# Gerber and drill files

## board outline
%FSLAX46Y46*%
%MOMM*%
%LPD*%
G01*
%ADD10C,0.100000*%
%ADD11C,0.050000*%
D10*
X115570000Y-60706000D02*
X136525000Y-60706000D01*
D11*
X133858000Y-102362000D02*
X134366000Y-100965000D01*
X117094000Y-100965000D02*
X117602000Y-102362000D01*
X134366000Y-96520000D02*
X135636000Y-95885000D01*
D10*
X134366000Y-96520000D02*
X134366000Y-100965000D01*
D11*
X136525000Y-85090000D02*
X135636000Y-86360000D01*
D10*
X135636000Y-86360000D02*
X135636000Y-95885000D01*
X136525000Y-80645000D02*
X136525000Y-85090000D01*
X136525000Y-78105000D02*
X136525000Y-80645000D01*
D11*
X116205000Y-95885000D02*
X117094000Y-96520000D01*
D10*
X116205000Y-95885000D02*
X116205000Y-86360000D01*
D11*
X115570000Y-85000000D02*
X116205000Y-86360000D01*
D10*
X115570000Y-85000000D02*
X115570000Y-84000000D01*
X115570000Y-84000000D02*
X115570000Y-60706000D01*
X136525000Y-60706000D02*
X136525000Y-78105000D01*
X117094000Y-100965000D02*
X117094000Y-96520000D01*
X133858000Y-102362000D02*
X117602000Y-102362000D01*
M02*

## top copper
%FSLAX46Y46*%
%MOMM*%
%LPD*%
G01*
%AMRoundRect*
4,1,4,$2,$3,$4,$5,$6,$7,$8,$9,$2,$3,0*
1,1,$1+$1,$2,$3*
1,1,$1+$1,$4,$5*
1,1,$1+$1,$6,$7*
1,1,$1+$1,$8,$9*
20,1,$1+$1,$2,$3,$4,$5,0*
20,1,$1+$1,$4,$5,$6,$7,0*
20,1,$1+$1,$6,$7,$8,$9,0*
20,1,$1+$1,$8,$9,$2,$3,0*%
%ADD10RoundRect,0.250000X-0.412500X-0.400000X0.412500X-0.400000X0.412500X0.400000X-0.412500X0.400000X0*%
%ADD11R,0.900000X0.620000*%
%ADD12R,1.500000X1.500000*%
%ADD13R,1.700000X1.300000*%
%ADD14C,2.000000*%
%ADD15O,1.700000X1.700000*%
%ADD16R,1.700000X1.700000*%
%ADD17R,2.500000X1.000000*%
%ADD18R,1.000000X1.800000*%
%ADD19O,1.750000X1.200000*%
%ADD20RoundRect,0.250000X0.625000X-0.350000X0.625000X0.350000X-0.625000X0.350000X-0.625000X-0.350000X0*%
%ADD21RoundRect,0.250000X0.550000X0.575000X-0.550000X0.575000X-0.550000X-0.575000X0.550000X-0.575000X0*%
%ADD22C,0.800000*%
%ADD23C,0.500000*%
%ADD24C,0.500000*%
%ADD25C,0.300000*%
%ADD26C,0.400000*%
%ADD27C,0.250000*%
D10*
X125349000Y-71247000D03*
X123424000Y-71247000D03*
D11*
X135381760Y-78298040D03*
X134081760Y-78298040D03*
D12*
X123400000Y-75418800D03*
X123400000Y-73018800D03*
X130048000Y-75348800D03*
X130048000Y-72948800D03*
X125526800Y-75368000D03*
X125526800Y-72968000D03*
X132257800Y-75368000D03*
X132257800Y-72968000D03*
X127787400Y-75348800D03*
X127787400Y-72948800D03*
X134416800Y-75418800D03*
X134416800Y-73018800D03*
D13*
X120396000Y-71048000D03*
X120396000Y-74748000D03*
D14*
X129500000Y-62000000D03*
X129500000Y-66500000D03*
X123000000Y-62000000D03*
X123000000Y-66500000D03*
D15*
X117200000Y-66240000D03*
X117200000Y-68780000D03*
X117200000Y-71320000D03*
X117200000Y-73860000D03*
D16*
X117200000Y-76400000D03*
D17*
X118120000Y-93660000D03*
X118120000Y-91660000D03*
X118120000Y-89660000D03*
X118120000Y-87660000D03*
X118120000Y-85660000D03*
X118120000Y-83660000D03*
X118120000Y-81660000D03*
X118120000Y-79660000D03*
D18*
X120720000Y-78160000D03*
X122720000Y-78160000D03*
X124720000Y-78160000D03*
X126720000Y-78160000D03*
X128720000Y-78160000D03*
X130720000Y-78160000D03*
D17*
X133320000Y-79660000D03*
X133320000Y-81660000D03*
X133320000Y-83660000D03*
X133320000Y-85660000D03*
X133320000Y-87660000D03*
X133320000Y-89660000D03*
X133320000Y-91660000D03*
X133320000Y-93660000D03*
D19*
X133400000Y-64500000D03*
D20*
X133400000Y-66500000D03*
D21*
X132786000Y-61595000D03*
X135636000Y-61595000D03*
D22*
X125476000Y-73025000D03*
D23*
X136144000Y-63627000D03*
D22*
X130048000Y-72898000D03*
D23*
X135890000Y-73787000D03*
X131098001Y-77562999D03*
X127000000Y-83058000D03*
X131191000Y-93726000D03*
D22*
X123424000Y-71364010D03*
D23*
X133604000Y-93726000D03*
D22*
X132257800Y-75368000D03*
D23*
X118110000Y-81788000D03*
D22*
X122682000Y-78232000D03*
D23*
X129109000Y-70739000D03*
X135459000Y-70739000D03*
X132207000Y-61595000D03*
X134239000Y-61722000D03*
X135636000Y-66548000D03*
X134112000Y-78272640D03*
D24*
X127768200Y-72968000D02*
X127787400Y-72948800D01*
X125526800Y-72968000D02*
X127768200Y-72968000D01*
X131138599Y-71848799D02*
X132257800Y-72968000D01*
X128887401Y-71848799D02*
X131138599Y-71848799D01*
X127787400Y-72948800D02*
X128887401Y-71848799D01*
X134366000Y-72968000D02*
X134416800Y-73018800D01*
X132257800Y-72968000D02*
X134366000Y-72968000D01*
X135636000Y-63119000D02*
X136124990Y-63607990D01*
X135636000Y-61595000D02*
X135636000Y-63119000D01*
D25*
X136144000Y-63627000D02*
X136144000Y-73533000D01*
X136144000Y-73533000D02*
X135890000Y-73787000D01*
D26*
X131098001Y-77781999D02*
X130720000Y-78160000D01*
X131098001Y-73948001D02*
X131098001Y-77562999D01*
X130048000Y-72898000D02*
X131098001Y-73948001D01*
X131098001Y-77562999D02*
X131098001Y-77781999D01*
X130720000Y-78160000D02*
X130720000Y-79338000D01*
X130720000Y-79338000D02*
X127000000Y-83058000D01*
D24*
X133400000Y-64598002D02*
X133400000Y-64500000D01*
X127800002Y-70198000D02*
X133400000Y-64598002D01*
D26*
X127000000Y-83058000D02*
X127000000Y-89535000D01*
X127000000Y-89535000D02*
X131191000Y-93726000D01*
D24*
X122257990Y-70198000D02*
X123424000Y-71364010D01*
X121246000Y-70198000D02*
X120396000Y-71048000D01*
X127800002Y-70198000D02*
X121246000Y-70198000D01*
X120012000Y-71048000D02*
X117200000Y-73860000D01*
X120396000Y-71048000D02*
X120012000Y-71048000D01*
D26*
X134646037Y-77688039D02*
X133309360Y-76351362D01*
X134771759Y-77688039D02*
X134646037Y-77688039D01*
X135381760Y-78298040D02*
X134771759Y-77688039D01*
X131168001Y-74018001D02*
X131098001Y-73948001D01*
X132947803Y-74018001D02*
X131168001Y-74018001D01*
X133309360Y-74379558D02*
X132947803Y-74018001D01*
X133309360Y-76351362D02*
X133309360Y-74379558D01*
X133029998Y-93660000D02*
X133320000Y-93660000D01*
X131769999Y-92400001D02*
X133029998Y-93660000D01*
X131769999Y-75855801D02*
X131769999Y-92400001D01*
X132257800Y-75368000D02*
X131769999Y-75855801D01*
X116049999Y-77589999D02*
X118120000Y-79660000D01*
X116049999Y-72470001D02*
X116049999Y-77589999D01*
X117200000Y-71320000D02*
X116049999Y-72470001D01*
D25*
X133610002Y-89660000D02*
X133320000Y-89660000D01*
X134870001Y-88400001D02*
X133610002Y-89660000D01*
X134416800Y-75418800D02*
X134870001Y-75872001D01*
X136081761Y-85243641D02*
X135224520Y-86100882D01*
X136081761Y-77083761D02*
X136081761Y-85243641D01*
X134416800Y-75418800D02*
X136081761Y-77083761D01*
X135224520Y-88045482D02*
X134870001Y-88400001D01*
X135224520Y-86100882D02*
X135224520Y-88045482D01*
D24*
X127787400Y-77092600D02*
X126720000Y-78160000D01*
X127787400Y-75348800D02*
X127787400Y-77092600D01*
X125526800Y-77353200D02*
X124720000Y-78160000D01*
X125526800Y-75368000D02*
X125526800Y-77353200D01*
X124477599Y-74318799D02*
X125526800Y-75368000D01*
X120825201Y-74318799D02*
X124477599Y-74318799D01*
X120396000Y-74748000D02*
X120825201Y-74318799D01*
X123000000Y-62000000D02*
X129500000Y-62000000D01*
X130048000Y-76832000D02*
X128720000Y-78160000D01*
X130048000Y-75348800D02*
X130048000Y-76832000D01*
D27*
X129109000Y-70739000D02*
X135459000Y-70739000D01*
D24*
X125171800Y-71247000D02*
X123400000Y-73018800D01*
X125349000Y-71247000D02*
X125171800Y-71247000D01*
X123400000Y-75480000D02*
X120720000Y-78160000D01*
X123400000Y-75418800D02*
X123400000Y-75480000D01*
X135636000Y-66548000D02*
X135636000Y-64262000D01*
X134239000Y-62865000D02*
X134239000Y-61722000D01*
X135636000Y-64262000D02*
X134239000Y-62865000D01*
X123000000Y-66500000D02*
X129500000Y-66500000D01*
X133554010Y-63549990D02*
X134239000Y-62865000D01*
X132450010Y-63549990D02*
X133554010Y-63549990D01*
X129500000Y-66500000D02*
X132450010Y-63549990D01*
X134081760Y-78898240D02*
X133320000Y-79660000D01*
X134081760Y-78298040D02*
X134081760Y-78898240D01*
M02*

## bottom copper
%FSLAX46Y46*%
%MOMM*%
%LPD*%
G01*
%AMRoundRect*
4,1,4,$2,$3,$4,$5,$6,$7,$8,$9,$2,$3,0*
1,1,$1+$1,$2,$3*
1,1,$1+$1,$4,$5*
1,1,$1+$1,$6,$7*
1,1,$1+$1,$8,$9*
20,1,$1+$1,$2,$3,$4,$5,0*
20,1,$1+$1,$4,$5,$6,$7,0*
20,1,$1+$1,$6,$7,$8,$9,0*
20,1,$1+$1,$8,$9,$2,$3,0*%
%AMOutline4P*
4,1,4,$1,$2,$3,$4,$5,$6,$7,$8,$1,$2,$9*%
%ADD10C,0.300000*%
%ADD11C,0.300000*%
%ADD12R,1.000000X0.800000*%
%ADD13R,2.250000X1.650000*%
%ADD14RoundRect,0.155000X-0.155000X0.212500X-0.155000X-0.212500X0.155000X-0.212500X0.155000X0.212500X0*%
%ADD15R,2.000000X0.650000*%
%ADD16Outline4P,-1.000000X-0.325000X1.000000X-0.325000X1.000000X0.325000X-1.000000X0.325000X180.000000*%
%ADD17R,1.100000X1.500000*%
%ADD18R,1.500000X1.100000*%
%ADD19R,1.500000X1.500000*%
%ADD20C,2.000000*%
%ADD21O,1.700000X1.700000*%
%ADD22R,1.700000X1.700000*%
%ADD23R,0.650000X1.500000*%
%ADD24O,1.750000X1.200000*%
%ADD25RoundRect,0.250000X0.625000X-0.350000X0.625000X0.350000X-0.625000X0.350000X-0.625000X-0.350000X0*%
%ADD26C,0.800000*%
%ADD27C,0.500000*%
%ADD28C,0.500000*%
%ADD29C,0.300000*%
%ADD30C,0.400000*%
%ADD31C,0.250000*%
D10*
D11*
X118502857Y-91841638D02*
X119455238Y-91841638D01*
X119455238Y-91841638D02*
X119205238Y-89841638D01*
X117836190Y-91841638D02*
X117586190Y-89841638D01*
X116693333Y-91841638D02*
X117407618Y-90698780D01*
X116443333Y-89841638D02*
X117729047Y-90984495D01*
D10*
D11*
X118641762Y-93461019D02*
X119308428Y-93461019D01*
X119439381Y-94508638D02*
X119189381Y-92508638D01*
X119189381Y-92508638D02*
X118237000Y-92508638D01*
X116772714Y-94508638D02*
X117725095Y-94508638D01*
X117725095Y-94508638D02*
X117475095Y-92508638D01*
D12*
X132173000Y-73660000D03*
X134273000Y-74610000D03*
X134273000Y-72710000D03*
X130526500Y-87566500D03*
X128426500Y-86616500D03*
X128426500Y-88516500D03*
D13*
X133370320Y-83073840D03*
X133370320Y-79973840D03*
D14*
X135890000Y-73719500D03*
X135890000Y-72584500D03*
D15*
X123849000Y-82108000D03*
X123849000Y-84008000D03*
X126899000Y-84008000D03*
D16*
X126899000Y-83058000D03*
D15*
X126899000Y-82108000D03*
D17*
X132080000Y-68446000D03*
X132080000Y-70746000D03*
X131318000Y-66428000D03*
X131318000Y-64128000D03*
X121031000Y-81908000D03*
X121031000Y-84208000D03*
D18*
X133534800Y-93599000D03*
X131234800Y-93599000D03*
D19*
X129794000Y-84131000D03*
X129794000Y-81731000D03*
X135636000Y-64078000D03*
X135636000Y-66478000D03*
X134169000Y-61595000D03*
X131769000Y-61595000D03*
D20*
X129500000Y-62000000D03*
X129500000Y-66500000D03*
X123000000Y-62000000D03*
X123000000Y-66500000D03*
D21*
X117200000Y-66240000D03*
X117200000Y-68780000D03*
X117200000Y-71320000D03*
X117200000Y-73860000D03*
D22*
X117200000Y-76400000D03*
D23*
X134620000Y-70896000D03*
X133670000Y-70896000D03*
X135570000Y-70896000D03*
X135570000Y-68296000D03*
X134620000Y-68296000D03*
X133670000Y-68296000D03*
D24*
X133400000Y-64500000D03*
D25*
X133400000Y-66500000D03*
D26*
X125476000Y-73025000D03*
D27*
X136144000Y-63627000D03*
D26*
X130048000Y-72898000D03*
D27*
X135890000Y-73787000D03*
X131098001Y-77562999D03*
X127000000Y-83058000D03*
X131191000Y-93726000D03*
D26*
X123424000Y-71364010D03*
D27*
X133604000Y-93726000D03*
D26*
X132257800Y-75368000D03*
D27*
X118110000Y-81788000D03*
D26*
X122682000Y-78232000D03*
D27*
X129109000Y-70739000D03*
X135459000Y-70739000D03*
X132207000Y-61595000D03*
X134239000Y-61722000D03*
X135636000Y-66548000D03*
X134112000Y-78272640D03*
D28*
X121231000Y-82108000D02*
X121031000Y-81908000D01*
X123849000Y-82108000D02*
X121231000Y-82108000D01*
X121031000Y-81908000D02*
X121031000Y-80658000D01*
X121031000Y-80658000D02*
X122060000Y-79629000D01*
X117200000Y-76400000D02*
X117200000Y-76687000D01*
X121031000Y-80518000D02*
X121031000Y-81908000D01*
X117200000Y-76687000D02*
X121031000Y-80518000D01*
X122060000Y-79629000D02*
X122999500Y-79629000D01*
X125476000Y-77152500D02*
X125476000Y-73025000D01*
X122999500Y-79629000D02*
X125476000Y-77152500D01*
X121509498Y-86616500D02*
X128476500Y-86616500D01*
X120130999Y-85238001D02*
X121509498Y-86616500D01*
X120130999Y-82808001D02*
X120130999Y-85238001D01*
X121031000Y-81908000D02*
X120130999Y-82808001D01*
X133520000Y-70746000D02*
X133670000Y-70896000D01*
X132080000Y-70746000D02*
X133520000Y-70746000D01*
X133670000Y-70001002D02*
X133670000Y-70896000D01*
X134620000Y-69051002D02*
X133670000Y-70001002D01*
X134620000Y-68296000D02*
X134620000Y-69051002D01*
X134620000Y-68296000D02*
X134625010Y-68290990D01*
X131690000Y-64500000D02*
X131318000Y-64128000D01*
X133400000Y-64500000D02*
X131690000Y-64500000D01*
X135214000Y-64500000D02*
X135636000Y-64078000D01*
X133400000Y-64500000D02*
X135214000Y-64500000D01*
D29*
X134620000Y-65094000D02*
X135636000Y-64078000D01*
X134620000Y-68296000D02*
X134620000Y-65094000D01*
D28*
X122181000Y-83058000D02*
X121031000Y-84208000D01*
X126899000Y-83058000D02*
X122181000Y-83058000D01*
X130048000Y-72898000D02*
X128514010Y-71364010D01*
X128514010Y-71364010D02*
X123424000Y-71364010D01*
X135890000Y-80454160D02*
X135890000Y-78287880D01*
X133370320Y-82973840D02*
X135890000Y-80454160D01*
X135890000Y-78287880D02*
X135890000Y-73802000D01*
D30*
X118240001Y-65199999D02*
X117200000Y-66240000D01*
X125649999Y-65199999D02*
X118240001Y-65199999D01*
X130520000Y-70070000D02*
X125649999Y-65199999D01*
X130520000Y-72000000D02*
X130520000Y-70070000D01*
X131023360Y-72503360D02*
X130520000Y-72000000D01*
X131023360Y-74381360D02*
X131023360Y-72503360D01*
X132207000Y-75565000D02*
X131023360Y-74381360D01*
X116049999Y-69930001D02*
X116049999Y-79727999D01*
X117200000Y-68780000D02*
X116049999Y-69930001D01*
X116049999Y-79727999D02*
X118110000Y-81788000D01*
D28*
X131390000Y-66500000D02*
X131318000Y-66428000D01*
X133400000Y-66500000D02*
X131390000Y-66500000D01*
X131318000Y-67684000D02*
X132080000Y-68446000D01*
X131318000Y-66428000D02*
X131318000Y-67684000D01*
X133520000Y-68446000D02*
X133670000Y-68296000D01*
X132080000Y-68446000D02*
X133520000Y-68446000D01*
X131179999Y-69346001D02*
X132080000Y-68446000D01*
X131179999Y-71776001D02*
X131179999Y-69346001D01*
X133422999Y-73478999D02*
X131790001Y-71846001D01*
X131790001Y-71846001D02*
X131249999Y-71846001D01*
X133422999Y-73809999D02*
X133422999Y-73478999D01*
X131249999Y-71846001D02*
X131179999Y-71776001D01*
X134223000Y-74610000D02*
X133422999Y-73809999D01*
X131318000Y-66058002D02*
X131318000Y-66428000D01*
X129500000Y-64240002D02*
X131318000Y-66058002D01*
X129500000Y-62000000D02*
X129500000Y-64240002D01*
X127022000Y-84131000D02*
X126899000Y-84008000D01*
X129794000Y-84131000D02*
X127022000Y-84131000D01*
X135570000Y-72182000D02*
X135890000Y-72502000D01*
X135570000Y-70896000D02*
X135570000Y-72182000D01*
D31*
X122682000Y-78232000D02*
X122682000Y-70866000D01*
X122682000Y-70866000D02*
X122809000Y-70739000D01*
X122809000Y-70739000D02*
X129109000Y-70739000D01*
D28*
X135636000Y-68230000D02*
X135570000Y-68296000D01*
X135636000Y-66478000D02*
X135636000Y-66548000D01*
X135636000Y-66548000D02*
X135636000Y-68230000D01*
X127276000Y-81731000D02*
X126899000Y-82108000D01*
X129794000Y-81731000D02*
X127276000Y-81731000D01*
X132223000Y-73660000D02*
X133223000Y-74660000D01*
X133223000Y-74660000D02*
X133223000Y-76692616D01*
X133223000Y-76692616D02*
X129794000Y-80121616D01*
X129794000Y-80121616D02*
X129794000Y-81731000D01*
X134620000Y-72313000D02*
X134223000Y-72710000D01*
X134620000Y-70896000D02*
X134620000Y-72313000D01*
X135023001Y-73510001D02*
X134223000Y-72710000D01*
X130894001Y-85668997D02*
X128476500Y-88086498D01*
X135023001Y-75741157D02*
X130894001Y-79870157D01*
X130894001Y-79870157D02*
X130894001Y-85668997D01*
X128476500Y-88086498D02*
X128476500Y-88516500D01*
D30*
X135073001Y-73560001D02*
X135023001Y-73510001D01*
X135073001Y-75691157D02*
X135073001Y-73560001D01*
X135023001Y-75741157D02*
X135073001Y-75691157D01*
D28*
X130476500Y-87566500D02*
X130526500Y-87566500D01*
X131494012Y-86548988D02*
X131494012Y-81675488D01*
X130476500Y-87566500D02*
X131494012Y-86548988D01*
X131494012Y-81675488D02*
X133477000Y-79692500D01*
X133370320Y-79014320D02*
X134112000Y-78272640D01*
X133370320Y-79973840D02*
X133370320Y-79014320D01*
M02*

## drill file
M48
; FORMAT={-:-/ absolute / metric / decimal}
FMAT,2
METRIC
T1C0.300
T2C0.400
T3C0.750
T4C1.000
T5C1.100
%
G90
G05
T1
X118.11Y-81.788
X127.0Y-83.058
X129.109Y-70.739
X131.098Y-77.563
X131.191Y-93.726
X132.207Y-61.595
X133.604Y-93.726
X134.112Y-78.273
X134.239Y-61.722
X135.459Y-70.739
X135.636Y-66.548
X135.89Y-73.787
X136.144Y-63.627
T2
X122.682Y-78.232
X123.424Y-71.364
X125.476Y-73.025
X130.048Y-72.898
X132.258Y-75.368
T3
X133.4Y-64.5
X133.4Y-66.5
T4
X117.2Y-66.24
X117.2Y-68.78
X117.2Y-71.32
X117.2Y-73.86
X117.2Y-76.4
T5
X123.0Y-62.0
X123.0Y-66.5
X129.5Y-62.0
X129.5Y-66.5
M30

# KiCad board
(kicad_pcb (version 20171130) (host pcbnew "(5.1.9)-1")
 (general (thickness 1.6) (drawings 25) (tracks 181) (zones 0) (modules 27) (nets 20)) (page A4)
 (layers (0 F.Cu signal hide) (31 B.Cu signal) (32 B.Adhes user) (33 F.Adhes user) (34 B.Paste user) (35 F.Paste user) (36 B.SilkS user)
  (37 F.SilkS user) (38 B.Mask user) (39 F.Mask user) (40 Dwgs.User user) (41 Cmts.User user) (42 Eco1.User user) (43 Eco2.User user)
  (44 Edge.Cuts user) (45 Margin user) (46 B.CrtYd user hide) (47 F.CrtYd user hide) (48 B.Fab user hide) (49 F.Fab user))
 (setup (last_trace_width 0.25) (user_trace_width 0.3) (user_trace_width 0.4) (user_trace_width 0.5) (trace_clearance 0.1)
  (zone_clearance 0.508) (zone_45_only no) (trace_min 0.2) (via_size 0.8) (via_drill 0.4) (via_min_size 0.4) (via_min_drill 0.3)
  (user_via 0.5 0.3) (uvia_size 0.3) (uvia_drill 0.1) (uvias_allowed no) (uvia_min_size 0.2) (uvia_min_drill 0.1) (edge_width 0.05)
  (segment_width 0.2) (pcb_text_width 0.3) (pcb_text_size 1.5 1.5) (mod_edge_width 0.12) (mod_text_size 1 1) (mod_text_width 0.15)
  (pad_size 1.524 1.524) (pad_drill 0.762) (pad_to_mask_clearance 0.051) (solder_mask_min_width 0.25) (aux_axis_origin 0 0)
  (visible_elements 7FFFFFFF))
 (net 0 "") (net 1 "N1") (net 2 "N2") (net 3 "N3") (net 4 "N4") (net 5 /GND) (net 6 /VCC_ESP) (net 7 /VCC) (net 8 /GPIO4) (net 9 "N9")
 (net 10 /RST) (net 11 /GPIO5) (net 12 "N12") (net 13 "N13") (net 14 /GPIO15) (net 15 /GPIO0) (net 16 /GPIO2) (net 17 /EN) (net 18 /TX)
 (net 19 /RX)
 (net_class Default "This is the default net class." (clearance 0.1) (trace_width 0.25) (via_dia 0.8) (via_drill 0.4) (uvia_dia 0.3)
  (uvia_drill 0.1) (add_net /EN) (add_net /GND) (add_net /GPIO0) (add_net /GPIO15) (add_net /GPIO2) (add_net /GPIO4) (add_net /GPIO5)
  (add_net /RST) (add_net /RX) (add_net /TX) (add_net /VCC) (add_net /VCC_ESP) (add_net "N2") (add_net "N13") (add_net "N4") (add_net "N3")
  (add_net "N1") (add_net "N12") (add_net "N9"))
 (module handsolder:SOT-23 (layer B.Cu) (at 133.223 73.66 180)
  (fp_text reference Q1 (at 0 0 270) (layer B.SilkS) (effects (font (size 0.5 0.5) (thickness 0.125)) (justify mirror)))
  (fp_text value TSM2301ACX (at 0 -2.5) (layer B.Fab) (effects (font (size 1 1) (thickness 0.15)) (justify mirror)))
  (pad 3 smd rect (at 1.05 0 180) (size 1 0.8) (layers B.Cu B.Paste B.Mask) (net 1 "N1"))
  (pad 2 smd rect (at -1.05 -0.95 180) (size 1 0.8) (layers B.Cu B.Paste B.Mask) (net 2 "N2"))
  (pad 1 smd rect (at -1.05 0.95 180) (size 1 0.8) (layers B.Cu B.Paste B.Mask) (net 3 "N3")))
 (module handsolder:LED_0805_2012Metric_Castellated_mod (layer F.Cu) (at 124.3865 71.247)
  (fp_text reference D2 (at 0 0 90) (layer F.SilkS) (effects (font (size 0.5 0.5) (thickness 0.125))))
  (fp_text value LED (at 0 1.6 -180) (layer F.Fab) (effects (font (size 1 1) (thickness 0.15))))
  (pad 2 smd roundrect (at 0.9625 0) (size 1.325 1.3) (layers F.Cu F.Paste F.Mask) (roundrect_rratio 0.1923076923076923) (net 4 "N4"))
  (pad 1 smd roundrect (at -0.9625 0) (size 1.325 1.3) (layers F.Cu F.Paste F.Mask) (roundrect_rratio 0.1923076923076923) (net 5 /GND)))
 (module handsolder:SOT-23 (layer B.Cu) (at 129.4765 87.5665)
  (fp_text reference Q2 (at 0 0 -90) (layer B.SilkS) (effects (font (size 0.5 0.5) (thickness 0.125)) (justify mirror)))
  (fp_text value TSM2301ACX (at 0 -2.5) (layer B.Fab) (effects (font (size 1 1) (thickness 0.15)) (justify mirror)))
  (pad 3 smd rect (at 1.05 0) (size 1 0.8) (layers B.Cu B.Paste B.Mask) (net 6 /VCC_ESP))
  (pad 2 smd rect (at -1.05 -0.95) (size 1 0.8) (layers B.Cu B.Paste B.Mask) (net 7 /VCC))
  (pad 1 smd rect (at -1.05 0.95) (size 1 0.8) (layers B.Cu B.Paste B.Mask) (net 3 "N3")))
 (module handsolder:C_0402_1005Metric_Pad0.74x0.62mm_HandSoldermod (layer F.Cu) (at 134.73176 78.29804)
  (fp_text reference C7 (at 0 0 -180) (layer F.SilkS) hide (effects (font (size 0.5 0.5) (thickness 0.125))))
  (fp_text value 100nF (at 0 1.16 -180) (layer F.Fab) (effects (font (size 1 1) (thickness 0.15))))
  (pad 2 smd rect (at 0.65 0) (size 0.9 0.62) (layers F.Cu F.Paste F.Mask) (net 5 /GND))
  (pad 1 smd rect (at -0.65 0) (size 0.9 0.62) (layers F.Cu F.Paste F.Mask) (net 6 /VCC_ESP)))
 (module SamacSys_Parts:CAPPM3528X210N (layer B.Cu) (at 133.37032 81.52384 270)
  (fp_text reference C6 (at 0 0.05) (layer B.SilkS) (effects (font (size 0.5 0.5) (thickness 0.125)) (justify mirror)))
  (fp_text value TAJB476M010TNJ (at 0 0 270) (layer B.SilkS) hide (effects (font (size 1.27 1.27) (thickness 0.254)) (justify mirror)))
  (pad 2 smd rect (at 1.55 0 270) (size 1.65 2.25) (layers B.Cu B.Paste B.Mask) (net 5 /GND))
  (pad 1 smd rect (at -1.55 0 270) (size 1.65 2.25) (layers B.Cu B.Paste B.Mask) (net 6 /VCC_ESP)))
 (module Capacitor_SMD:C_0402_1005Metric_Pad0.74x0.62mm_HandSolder (layer B.Cu) (at 135.89 73.152 270)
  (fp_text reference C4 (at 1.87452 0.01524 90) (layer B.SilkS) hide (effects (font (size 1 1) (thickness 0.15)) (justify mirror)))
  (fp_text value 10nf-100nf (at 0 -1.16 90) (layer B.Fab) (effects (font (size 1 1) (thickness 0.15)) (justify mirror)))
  (pad 2 smd roundrect (at 0.5675 0 270) (size 0.735 0.62) (layers B.Cu B.Paste B.Mask) (roundrect_rratio 0.25) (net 5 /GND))
  (pad 1 smd roundrect (at -0.5675 0 270) (size 0.735 0.62) (layers B.Cu B.Paste B.Mask) (roundrect_rratio 0.25) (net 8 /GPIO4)))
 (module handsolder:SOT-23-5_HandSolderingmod (layer B.Cu) (at 125.349 83.058 180)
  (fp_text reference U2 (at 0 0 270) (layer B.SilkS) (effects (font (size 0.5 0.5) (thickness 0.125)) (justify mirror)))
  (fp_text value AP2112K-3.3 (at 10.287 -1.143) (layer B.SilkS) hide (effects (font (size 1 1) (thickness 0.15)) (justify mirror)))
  (pad 5 smd rect (at 1.5 0.95 180) (size 2 0.65) (layers B.Cu B.Paste B.Mask) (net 7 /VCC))
  (pad 4 smd rect (at 1.5 -0.95 180) (size 2 0.65) (layers B.Cu B.Paste B.Mask))
  (pad 3 smd rect (at -1.55 -0.95 180) (size 2 0.65) (layers B.Cu B.Paste B.Mask) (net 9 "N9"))
  (pad 2 smd trapezoid (at -1.55 0 180) (size 2 0.65) (layers B.Cu B.Paste B.Mask) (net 5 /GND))
  (pad 1 smd rect (at -1.55 0.95 180) (size 2 0.65) (layers B.Cu B.Paste B.Mask) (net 1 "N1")))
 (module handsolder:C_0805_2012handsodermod (layer B.Cu) (at 132.08 69.596 90)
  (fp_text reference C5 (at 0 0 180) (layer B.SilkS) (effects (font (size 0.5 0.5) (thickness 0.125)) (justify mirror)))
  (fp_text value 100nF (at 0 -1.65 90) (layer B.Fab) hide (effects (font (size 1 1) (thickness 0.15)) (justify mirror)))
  (pad 2 smd rect (at 1.15 0 90) (size 1.5 1.1) (layers B.Cu B.Paste B.Mask) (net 2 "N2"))
  (pad 1 smd rect (at -1.15 0 90) (size 1.5 1.1) (layers B.Cu B.Paste B.Mask) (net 5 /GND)))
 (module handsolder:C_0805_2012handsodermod (layer B.Cu) (at 131.318 65.278 270)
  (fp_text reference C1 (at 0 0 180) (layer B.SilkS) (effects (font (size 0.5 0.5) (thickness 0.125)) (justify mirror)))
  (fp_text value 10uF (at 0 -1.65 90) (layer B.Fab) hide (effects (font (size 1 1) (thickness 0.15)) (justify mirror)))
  (pad 2 smd rect (at 1.15 0 270) (size 1.5 1.1) (layers B.Cu B.Paste B.Mask) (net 2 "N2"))
  (pad 1 smd rect (at -1.15 0 270) (size 1.5 1.1) (layers B.Cu B.Paste B.Mask) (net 5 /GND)))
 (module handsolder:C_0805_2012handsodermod (layer B.Cu) (at 121.031 83.058 90)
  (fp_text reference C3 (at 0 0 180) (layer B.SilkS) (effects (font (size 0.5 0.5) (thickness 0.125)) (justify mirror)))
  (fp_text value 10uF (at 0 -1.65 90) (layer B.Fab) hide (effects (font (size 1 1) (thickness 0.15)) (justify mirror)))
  (pad 2 smd rect (at 1.15 0 90) (size 1.5 1.1) (layers B.Cu B.Paste B.Mask) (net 7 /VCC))
  (pad 1 smd rect (at -1.15 0 90) (size 1.5 1.1) (layers B.Cu B.Paste B.Mask) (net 5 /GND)))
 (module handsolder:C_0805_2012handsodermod (layer B.Cu) (at 132.3848 93.599)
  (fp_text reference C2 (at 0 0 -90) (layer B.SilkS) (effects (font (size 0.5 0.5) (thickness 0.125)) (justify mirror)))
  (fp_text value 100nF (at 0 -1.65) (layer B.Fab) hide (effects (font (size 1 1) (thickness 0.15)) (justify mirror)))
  (pad 2 smd rect (at 1.15 0) (size 1.5 1.1) (layers B.Cu B.Paste B.Mask) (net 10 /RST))
  (pad 1 smd rect (at -1.15 0) (size 1.5 1.1) (layers B.Cu B.Paste B.Mask) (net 5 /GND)))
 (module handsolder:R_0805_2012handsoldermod (layer F.Cu) (at 123.4 74.2188 270)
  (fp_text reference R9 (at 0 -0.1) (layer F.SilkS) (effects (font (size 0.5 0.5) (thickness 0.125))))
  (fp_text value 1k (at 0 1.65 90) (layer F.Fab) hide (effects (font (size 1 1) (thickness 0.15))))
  (pad 2 smd rect (at 1.2 0 270) (size 1.5 1.5) (layers F.Cu F.Paste F.Mask) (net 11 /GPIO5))
  (pad 1 smd rect (at -1.2 0 270) (size 1.5 1.5) (layers F.Cu F.Paste F.Mask) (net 4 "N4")))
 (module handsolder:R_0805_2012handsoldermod (layer B.Cu) (at 129.794 82.931 270)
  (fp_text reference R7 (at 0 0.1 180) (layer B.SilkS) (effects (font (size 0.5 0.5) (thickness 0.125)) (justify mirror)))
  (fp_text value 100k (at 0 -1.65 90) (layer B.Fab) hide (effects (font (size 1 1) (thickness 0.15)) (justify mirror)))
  (pad 2 smd rect (at 1.2 0 270) (size 1.5 1.5) (layers B.Cu B.Paste B.Mask) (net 9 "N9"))
  (pad 1 smd rect (at -1.2 0 270) (size 1.5 1.5) (layers B.Cu B.Paste B.Mask) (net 1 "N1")))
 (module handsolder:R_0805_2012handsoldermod (layer B.Cu) (at 135.636 65.278 90)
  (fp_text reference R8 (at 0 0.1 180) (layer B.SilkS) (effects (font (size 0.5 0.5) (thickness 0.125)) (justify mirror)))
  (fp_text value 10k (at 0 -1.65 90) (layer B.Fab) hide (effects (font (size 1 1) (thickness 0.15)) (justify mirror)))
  (pad 2 smd rect (at 1.2 0 90) (size 1.5 1.5) (layers B.Cu B.Paste B.Mask) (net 5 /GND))
  (pad 1 smd rect (at -1.2 0 90) (size 1.5 1.5) (layers B.Cu B.Paste B.Mask) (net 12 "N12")))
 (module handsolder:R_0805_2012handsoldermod (layer B.Cu) (at 132.969 61.595)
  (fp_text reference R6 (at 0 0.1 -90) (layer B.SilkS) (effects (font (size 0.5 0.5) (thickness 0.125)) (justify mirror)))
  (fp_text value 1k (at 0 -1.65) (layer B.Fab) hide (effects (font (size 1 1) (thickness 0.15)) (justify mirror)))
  (pad 2 smd rect (at 1.2 0) (size 1.5 1.5) (layers B.Cu B.Paste B.Mask) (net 12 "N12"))
  (pad 1 smd rect (at -1.2 0) (size 1.5 1.5) (layers B.Cu B.Paste B.Mask) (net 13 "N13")))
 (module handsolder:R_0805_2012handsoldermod (layer F.Cu) (at 130.048 74.1488 270)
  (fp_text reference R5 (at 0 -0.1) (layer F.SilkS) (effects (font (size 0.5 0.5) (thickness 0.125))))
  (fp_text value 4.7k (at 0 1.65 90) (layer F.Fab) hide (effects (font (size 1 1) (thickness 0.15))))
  (pad 2 smd rect (at 1.2 0 270) (size 1.5 1.5) (layers F.Cu F.Paste F.Mask) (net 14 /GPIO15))
  (pad 1 smd rect (at -1.2 0 270) (size 1.5 1.5) (layers F.Cu F.Paste F.Mask) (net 5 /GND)))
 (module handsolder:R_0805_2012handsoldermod (layer F.Cu) (at 125.5268 74.168 270)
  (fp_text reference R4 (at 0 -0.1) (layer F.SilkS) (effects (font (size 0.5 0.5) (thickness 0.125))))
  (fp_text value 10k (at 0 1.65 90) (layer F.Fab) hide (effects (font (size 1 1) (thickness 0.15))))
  (pad 2 smd rect (at 1.2 0 270) (size 1.5 1.5) (layers F.Cu F.Paste F.Mask) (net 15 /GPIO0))
  (pad 1 smd rect (at -1.2 0 270) (size 1.5 1.5) (layers F.Cu F.Paste F.Mask) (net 7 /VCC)))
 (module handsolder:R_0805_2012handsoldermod (layer F.Cu) (at 132.2578 74.168 270)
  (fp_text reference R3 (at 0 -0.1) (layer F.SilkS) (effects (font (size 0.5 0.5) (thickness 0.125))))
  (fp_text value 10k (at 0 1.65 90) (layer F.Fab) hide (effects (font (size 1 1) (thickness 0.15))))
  (pad 2 smd rect (at 1.2 0 270) (size 1.5 1.5) (layers F.Cu F.Paste F.Mask) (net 10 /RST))
  (pad 1 smd rect (at -1.2 0 270) (size 1.5 1.5) (layers F.Cu F.Paste F.Mask) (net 7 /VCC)))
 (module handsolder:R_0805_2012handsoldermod (layer F.Cu) (at 127.7874 74.1488 270)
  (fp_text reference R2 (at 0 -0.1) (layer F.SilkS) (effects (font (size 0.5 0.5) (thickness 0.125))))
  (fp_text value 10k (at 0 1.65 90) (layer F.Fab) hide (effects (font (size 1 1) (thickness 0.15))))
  (pad 2 smd rect (at 1.2 0 270) (size 1.5 1.5) (layers F.Cu F.Paste F.Mask) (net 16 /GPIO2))
  (pad 1 smd rect (at -1.2 0 270) (size 1.5 1.5) (layers F.Cu F.Paste F.Mask) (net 7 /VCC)))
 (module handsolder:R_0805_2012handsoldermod (layer F.Cu) (at 134.4168 74.2188 270)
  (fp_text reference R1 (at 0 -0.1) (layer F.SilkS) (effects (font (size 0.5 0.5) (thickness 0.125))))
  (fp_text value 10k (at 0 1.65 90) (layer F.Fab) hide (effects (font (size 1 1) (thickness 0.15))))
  (pad 2 smd rect (at 1.2 0 270) (size 1.5 1.5) (layers F.Cu F.Paste F.Mask) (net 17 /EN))
  (pad 1 smd rect (at -1.2 0 270) (size 1.5 1.5) (layers F.Cu F.Paste F.Mask) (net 7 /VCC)))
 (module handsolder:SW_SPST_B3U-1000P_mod (layer F.Cu) (at 120.396 72.898 90)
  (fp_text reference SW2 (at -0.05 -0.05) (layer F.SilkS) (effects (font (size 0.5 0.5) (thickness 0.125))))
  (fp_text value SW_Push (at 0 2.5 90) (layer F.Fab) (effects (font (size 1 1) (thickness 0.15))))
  (pad 2 smd rect (at 1.85 0 90) (size 1.3 1.7) (layers F.Cu F.Paste F.Mask) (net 5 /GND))
  (pad 1 smd rect (at -1.85 0 90) (size 1.3 1.7) (layers F.Cu F.Paste F.Mask) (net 15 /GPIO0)))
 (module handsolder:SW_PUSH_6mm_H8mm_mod (layer F.Cu) (at 123 62)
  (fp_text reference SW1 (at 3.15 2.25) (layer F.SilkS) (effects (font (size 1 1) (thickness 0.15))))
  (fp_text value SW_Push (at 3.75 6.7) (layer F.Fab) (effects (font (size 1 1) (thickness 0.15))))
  (pad 1 thru_hole circle (at 6.5 0 90) (size 2 2) (drill 1.1) (layers *.Cu *.Mask) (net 2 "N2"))
  (pad 2 thru_hole circle (at 6.5 4.5 90) (size 2 2) (drill 1.1) (layers *.Cu *.Mask) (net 12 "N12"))
  (pad 1 thru_hole circle (at 0 0 90) (size 2 2) (drill 1.1) (layers *.Cu *.Mask) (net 2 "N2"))
  (pad 2 thru_hole circle (at 0 4.5 90) (size 2 2) (drill 1.1) (layers *.Cu *.Mask) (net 12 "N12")))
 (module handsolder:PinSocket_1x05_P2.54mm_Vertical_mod (layer F.Cu) (at 117.2 76.4 180)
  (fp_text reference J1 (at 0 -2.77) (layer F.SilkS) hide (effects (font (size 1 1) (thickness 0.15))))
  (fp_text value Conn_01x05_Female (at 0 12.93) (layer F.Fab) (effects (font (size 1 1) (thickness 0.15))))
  (pad 5 thru_hole oval (at 0 10.16 180) (size 1.7 1.7) (drill 1) (layers *.Cu *.Mask) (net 10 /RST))
  (pad 4 thru_hole oval (at 0 7.62 180) (size 1.7 1.7) (drill 1) (layers *.Cu *.Mask) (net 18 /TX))
  (pad 3 thru_hole oval (at 0 5.08 180) (size 1.7 1.7) (drill 1) (layers *.Cu *.Mask) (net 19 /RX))
  (pad 2 thru_hole oval (at 0 2.54 180) (size 1.7 1.7) (drill 1) (layers *.Cu *.Mask) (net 5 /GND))
  (pad 1 thru_hole rect (at 0 0 180) (size 1.7 1.7) (drill 1) (layers *.Cu *.Mask) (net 7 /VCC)))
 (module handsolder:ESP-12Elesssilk (layer F.Cu) (at 125.72 90.16 180)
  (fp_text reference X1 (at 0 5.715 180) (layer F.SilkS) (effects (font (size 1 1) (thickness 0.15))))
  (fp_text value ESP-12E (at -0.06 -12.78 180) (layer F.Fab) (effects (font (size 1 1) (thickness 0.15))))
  (pad 22 smd rect (at 7.6 -3.5 180) (size 2.5 1) (layers F.Cu F.Paste F.Mask))
  (pad 21 smd rect (at 7.6 -1.5 180) (size 2.5 1) (layers F.Cu F.Paste F.Mask))
  (pad 20 smd rect (at 7.6 0.5 180) (size 2.5 1) (layers F.Cu F.Paste F.Mask))
  (pad 19 smd rect (at 7.6 2.5 180) (size 2.5 1) (layers F.Cu F.Paste F.Mask))
  (pad 18 smd rect (at 7.6 4.5 180) (size 2.5 1) (layers F.Cu F.Paste F.Mask))
  (pad 17 smd rect (at 7.6 6.5 180) (size 2.5 1) (layers F.Cu F.Paste F.Mask))
  (pad 16 smd rect (at 7.6 8.5 180) (size 2.5 1) (layers F.Cu F.Paste F.Mask) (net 18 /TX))
  (pad 15 smd rect (at 7.6 10.5 180) (size 2.5 1) (layers F.Cu F.Paste F.Mask) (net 19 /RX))
  (pad 14 smd rect (at 5 12 180) (size 1 1.8) (layers F.Cu F.Paste F.Mask) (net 11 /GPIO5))
  (pad 13 smd rect (at 3 12 180) (size 1 1.8) (layers F.Cu F.Paste F.Mask) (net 8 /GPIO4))
  (pad 12 smd rect (at 1 12 180) (size 1 1.8) (layers F.Cu F.Paste F.Mask) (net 15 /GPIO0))
  (pad 11 smd rect (at -1 12 180) (size 1 1.8) (layers F.Cu F.Paste F.Mask) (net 16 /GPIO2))
  (pad 10 smd rect (at -3 12 180) (size 1 1.8) (layers F.Cu F.Paste F.Mask) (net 14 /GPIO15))
  (pad 9 smd rect (at -5 12 180) (size 1 1.8) (layers F.Cu F.Paste F.Mask) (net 5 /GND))
  (pad 8 smd rect (at -7.6 10.5 180) (size 2.5 1) (layers F.Cu F.Paste F.Mask) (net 6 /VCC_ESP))
  (pad 7 smd rect (at -7.6 8.5 180) (size 2.5 1) (layers F.Cu F.Paste F.Mask))
  (pad 6 smd rect (at -7.6 6.5 180) (size 2.5 1) (layers F.Cu F.Paste F.Mask))
  (pad 5 smd rect (at -7.6 4.5 180) (size 2.5 1) (layers F.Cu F.Paste F.Mask))
  (pad 4 smd rect (at -7.6 2.5 180) (size 2.5 1) (layers F.Cu F.Paste F.Mask))
  (pad 3 smd rect (at -7.6 0.5 180) (size 2.5 1) (layers F.Cu F.Paste F.Mask) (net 17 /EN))
  (pad 2 smd rect (at -7.6 -1.5 180) (size 2.5 1) (layers F.Cu F.Paste F.Mask))
  (pad 1 smd rect (at -7.6 -3.5 180) (size 2.5 1) (layers F.Cu F.Paste F.Mask) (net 10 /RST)))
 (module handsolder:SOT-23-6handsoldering (layer B.Cu) (at 134.62 69.596 270)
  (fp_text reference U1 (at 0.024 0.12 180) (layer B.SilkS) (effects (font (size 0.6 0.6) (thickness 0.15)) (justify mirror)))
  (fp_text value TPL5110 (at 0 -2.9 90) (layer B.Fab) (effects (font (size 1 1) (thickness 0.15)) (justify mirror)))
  (pad 5 smd rect (at 1.3 0 270) (size 1.5 0.65) (layers B.Cu B.Paste B.Mask) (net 3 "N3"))
  (pad 6 smd rect (at 1.3 0.95 270) (size 1.5 0.65) (layers B.Cu B.Paste B.Mask) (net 5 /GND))
  (pad 4 smd rect (at 1.3 -0.95 270) (size 1.5 0.65) (layers B.Cu B.Paste B.Mask) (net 8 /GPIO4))
  (pad 3 smd rect (at -1.3 -0.95 270) (size 1.5 0.65) (layers B.Cu B.Paste B.Mask) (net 12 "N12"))
  (pad 2 smd rect (at -1.3 0 270) (size 1.5 0.65) (layers B.Cu B.Paste B.Mask) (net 5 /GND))
  (pad 1 smd rect (at -1.3 0.95 270) (size 1.5 0.65) (layers B.Cu B.Paste B.Mask) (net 2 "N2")))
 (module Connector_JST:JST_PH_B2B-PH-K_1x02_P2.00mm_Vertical (layer F.Cu) (at 133.4 66.5 90)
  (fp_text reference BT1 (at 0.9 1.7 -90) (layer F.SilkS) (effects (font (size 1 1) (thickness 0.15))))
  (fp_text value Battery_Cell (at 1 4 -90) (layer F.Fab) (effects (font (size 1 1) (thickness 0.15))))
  (pad 2 thru_hole oval (at 2 0 90) (size 1.2 1.75) (drill 0.75) (layers *.Cu *.Mask) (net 5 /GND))
  (pad 1 thru_hole roundrect (at 0 0 90) (size 1.2 1.75) (drill 0.75) (layers *.Cu *.Mask) (roundrect_rratio 0.208333) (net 2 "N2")))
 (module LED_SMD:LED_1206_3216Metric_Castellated (layer F.Cu) (at 134.211 61.595 180)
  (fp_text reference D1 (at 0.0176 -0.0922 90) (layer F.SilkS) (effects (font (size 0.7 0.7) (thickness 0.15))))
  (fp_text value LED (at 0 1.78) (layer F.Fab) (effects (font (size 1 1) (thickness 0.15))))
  (pad 2 smd roundrect (at 1.425 0 180) (size 1.6 1.65) (layers F.Cu F.Paste F.Mask) (roundrect_rratio 0.15625) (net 13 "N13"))
  (pad 1 smd roundrect (at -1.425 0 180) (size 1.6 1.65) (layers F.Cu F.Paste F.Mask) (roundrect_rratio 0.15625) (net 5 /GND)))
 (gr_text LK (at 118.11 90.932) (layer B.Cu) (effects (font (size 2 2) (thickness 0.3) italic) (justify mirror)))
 (gr_line (start 115.57 60.706) (end 136.525 60.706) (layer Edge.Cuts) (width 0.1))
 (gr_line (start 133.858 102.362) (end 134.366 100.965) (layer Edge.Cuts) (width 0.05))
 (gr_line (start 117.094 100.965) (end 117.602 102.362) (layer Edge.Cuts) (width 0.05))
 (gr_line (start 134.366 96.52) (end 135.636 95.885) (layer Edge.Cuts) (width 0.05))
 (gr_line (start 134.366 96.52) (end 134.366 100.965) (layer Edge.Cuts) (width 0.1))
 (gr_line (start 136.525 85.09) (end 135.636 86.36) (layer Edge.Cuts) (width 0.05))
 (gr_line (start 135.636 86.36) (end 135.636 95.885) (layer Edge.Cuts) (width 0.1))
 (gr_line (start 136.525 80.645) (end 136.525 85.09) (layer Edge.Cuts) (width 0.1))
 (gr_line (start 136.525 78.105) (end 136.525 80.645) (layer Edge.Cuts) (width 0.1))
 (gr_line (start 116.205 95.885) (end 117.094 96.52) (layer Edge.Cuts) (width 0.05))
 (gr_line (start 116.205 95.885) (end 116.205 86.36) (layer Edge.Cuts) (width 0.1))
 (gr_line (start 115.57 85) (end 116.205 86.36) (layer Edge.Cuts) (width 0.05))
 (gr_line (start 115.57 85) (end 115.57 84) (layer Edge.Cuts) (width 0.1))
 (gr_line (start 115.57 84) (end 115.57 60.706) (layer Edge.Cuts) (width 0.1))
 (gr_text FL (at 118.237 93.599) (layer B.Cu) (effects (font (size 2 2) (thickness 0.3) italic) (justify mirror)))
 (gr_line (start 136.525 60.706) (end 136.525 78.105) (layer Edge.Cuts) (width 0.1))
 (gr_line (start 117.094 100.965) (end 117.094 96.52) (layer Edge.Cuts) (width 0.1))
 (gr_line (start 133.858 102.362) (end 117.602 102.362) (layer Edge.Cuts) (width 0.1))
 (via (at 125.476 73.025) (size 0.8) (drill 0.4) (layers F.Cu B.Cu) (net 7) (status 30))
 (segment (start 121.231 82.108) (end 121.031 81.908) (width 0.5) (layer B.Cu) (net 7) (status 30))
 (segment (start 123.849 82.108) (end 121.231 82.108) (width 0.5) (layer B.Cu) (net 7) (status 30))
 (segment (start 121.031 81.908) (end 121.031 80.658) (width 0.5) (layer B.Cu) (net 7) (status 10))
 (segment (start 121.031 80.658) (end 122.06 79.629) (width 0.5) (layer B.Cu) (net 7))
 (segment (start 127.7682 72.968) (end 127.7874 72.9488) (width 0.5) (layer F.Cu) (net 7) (status 30))
 (segment (start 125.5268 72.968) (end 127.7682 72.968) (width 0.5) (layer F.Cu) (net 7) (status 30))
 (segment (start 131.138599 71.848799) (end 132.2578 72.968) (width 0.5) (layer F.Cu) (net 7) (status 20))
 (segment (start 128.887401 71.848799) (end 131.138599 71.848799) (width 0.5) (layer F.Cu) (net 7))
 (segment (start 127.7874 72.9488) (end 128.887401 71.848799) (width 0.5) (layer F.Cu) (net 7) (status 10))
 (segment (start 134.366 72.968) (end 134.4168 73.0188) (width 0.5) (layer F.Cu) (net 7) (status 30))
 (segment (start 132.2578 72.968) (end 134.366 72.968) (width 0.5) (layer F.Cu) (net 7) (status 30))
 (segment (start 117.2 76.4) (end 117.2 76.687) (width 0.5) (layer B.Cu) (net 7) (status 30))
 (segment (start 121.031 80.518) (end 121.031 81.908) (width 0.5) (layer B.Cu) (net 7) (status 20))
 (segment (start 117.2 76.687) (end 121.031 80.518) (width 0.5) (layer B.Cu) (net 7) (status 10))
 (segment (start 122.06 79.629) (end 122.9995 79.629) (width 0.5) (layer B.Cu) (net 7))
 (segment (start 125.476 77.1525) (end 125.476 73.025) (width 0.5) (layer B.Cu) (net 7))
 (segment (start 122.9995 79.629) (end 125.476 77.1525) (width 0.5) (layer B.Cu) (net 7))
 (segment (start 121.509498 86.6165) (end 128.4765 86.6165) (width 0.5) (layer B.Cu) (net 7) (status 20))
 (segment (start 120.130999 85.238001) (end 121.509498 86.6165) (width 0.5) (layer B.Cu) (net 7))
 (segment (start 120.130999 82.808001) (end 120.130999 85.238001) (width 0.5) (layer B.Cu) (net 7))
 (segment (start 121.031 81.908) (end 120.130999 82.808001) (width 0.5) (layer B.Cu) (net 7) (status 10))
 (via (at 136.144 63.627) (size 0.5) (drill 0.3) (layers F.Cu B.Cu) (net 5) (status 30))
 (segment (start 133.52 70.746) (end 133.67 70.896) (width 0.5) (layer B.Cu) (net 5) (status 30))
 (segment (start 132.08 70.746) (end 133.52 70.746) (width 0.5) (layer B.Cu) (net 5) (status 30))
 (segment (start 133.67 70.001002) (end 133.67 70.896) (width 0.5) (layer B.Cu) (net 5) (status 20))
 (segment (start 134.62 69.051002) (end 133.67 70.001002) (width 0.5) (layer B.Cu) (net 5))
 (segment (start 134.62 68.296) (end 134.62 69.051002) (width 0.5) (layer B.Cu) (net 5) (status 10))
 (segment (start 134.62 68.296) (end 134.62501 68.29099) (width 0.5) (layer B.Cu) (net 5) (status 30))
 (segment (start 131.69 64.5) (end 131.318 64.128) (width 0.5) (layer B.Cu) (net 5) (status 30))
 (segment (start 133.4 64.5) (end 131.69 64.5) (width 0.5) (layer B.Cu) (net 5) (status 30))
 (segment (start 135.214 64.5) (end 135.636 64.078) (width 0.5) (layer B.Cu) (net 5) (status 30))
 (segment (start 133.4 64.5) (end 135.214 64.5) (width 0.5) (layer B.Cu) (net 5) (status 30))
 (segment (start 134.62 65.094) (end 135.636 64.078) (width 0.3) (layer B.Cu) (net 5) (status 20))
 (segment (start 134.62 68.296) (end 134.62 65.094) (width 0.3) (layer B.Cu) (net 5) (status 10))
 (segment (start 122.181 83.058) (end 121.031 84.208) (width 0.5) (layer B.Cu) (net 5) (status 20))
 (segment (start 126.899 83.058) (end 122.181 83.058) (width 0.5) (layer B.Cu) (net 5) (status 10))
 (segment (start 135.636 63.119) (end 136.12499 63.60799) (width 0.5) (layer F.Cu) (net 5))
 (segment (start 135.636 61.595) (end 135.636 63.119) (width 0.5) (layer F.Cu) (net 5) (status 10))
 (via (at 130.048 72.898) (size 0.8) (drill 0.4) (layers F.Cu B.Cu) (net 5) (status 30))
 (segment (start 136.144 63.627) (end 136.144 73.533) (width 0.3) (layer F.Cu) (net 5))
 (segment (start 136.144 73.533) (end 135.89 73.787) (width 0.3) (layer F.Cu) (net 5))
 (via (at 135.89 73.787) (size 0.5) (drill 0.3) (layers F.Cu B.Cu) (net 5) (status 30))
 (segment (start 131.098001 77.781999) (end 130.72 78.16) (width 0.4) (layer F.Cu) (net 5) (status 30))
 (segment (start 131.098001 73.948001) (end 131.098001 77.562999) (width 0.4) (layer F.Cu) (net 5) (status 20))
 (segment (start 130.048 72.898) (end 131.098001 73.948001) (width 0.4) (layer F.Cu) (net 5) (status 10))
 (segment (start 131.098001 77.562999) (end 131.098001 77.781999) (width 0.4) (layer F.Cu) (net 5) (status 30))
 (via (at 131.098001 77.562999) (size 0.5) (drill 0.3) (layers F.Cu B.Cu) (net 5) (status 30))
 (segment (start 130.72 78.16) (end 130.72 79.338) (width 0.4) (layer F.Cu) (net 5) (status 10))
 (segment (start 130.72 79.338) (end 127 83.058) (width 0.4) (layer F.Cu) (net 5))
 (via (at 127 83.058) (size 0.5) (drill 0.3) (layers F.Cu B.Cu) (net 5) (status 30))
 (segment (start 133.4 64.598002) (end 133.4 64.5) (width 0.5) (layer F.Cu) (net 5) (status 30))
 (segment (start 127.800002 70.198) (end 133.4 64.598002) (width 0.5) (layer F.Cu) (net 5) (status 20))
 (via (at 131.191 93.726) (size 0.5) (drill 0.3) (layers F.Cu B.Cu) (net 5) (status 30))
 (segment (start 127 83.058) (end 127 89.535) (width 0.4) (layer F.Cu) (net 5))
 (segment (start 127 89.535) (end 131.191 93.726) (width 0.4) (layer F.Cu) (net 5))
 (via (at 123.424 71.36401) (size 0.8) (drill 0.4) (layers F.Cu B.Cu) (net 5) (status 30))
 (segment (start 122.25799 70.198) (end 123.424 71.36401) (width 0.5) (layer F.Cu) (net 5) (status 20))
 (segment (start 130.048 72.898) (end 128.51401 71.36401) (width 0.5) (layer B.Cu) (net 5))
 (segment (start 128.51401 71.36401) (end 123.424 71.36401) (width 0.5) (layer B.Cu) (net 5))
 (segment (start 121.246 70.198) (end 120.396 71.048) (width 0.5) (layer F.Cu) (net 5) (status 20))
 (segment (start 127.800002 70.198) (end 121.246 70.198) (width 0.5) (layer F.Cu) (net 5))
 (segment (start 120.012 71.048) (end 117.2 73.86) (width 0.5) (layer F.Cu) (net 5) (status 30))
 (segment (start 120.396 71.048) (end 120.012 71.048) (width 0.5) (layer F.Cu) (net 5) (status 30))
 (segment (start 135.89 80.45416) (end 135.89 78.28788) (width 0.5) (layer B.Cu) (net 5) (status 20))
 (segment (start 133.37032 82.97384) (end 135.89 80.45416) (width 0.5) (layer B.Cu) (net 5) (status 10))
 (segment (start 135.89 78.28788) (end 135.89 73.802) (width 0.5) (layer B.Cu) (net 5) (status 20))
 (segment (start 134.646037 77.688039) (end 133.30936 76.351362) (width 0.4) (layer F.Cu) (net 5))
 (segment (start 134.771759 77.688039) (end 134.646037 77.688039) (width 0.4) (layer F.Cu) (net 5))
 (segment (start 135.38176 78.29804) (end 134.771759 77.688039) (width 0.4) (layer F.Cu) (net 5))
 (segment (start 131.168001 74.018001) (end 131.098001 73.948001) (width 0.4) (layer F.Cu) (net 5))
 (segment (start 132.947803 74.018001) (end 131.168001 74.018001) (width 0.4) (layer F.Cu) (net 5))
 (segment (start 133.30936 74.379558) (end 132.947803 74.018001) (width 0.4) (layer F.Cu) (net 5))
 (segment (start 133.30936 76.351362) (end 133.30936 74.379558) (width 0.4) (layer F.Cu) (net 5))
 (via (at 133.604 93.726) (size 0.5) (drill 0.3) (layers F.Cu B.Cu) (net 10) (status 30))
 (segment (start 133.029998 93.66) (end 133.32 93.66) (width 0.4) (layer F.Cu) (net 10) (status 30))
 (segment (start 131.769999 92.400001) (end 133.029998 93.66) (width 0.4) (layer F.Cu) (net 10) (status 20))
 (segment (start 131.769999 75.855801) (end 131.769999 92.400001) (width 0.4) (layer F.Cu) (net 10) (status 10))
 (segment (start 132.2578 75.368) (end 131.769999 75.855801) (width 0.4) (layer F.Cu) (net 10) (status 30))
 (via (at 132.2578 75.368) (size 0.8) (drill 0.4) (layers F.Cu B.Cu) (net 10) (status 30))
 (segment (start 118.240001 65.199999) (end 117.2 66.24) (width 0.4) (layer B.Cu) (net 10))
 (segment (start 125.649999 65.199999) (end 118.240001 65.199999) (width 0.4) (layer B.Cu) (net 10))
 (segment (start 130.52 70.07) (end 125.649999 65.199999) (width 0.4) (layer B.Cu) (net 10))
 (segment (start 130.52 72) (end 130.52 70.07) (width 0.4) (layer B.Cu) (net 10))
 (segment (start 131.02336 72.50336) (end 130.52 72) (width 0.4) (layer B.Cu) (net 10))
 (segment (start 131.02336 74.38136) (end 131.02336 72.50336) (width 0.4) (layer B.Cu) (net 10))
 (segment (start 132.207 75.565) (end 131.02336 74.38136) (width 0.4) (layer B.Cu) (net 10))
 (segment (start 116.049999 77.589999) (end 118.12 79.66) (width 0.4) (layer F.Cu) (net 19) (status 20))
 (segment (start 116.049999 72.470001) (end 116.049999 77.589999) (width 0.4) (layer F.Cu) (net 19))
 (segment (start 117.2 71.32) (end 116.049999 72.470001) (width 0.4) (layer F.Cu) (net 19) (status 10))
 (segment (start 116.049999 69.930001) (end 116.049999 79.727999) (width 0.4) (layer B.Cu) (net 18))
 (segment (start 117.2 68.78) (end 116.049999 69.930001) (width 0.4) (layer B.Cu) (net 18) (status 10))
 (segment (start 116.049999 79.727999) (end 118.11 81.788) (width 0.4) (layer B.Cu) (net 18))
 (via (at 118.11 81.788) (size 0.5) (drill 0.3) (layers F.Cu B.Cu) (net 18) (status 30))
 (segment (start 133.610002 89.66) (end 133.32 89.66) (width 0.3) (layer F.Cu) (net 17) (status 30))
 (segment (start 134.870001 88.400001) (end 133.610002 89.66) (width 0.3) (layer F.Cu) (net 17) (status 20))
 (segment (start 134.4168 75.4188) (end 134.870001 75.872001) (width 0.3) (layer F.Cu) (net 17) (status 30))
 (segment (start 136.081761 85.243641) (end 135.22452 86.100882) (width 0.3) (layer F.Cu) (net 17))
 (segment (start 136.081761 77.083761) (end 136.081761 85.243641) (width 0.3) (layer F.Cu) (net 17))
 (segment (start 134.4168 75.4188) (end 136.081761 77.083761) (width 0.3) (layer F.Cu) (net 17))
 (segment (start 135.22452 88.045482) (end 134.870001 88.400001) (width 0.3) (layer F.Cu) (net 17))
 (segment (start 135.22452 86.100882) (end 135.22452 88.045482) (width 0.3) (layer F.Cu) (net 17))
 (segment (start 127.7874 77.0926) (end 126.72 78.16) (width 0.5) (layer F.Cu) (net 16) (status 20))
 (segment (start 127.7874 75.3488) (end 127.7874 77.0926) (width 0.5) (layer F.Cu) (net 16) (status 10))
 (segment (start 125.5268 77.3532) (end 124.72 78.16) (width 0.5) (layer F.Cu) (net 15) (status 20))
 (segment (start 125.5268 75.368) (end 125.5268 77.3532) (width 0.5) (layer F.Cu) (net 15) (status 10))
 (segment (start 124.477599 74.318799) (end 125.5268 75.368) (width 0.5) (layer F.Cu) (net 15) (status 20))
 (segment (start 120.825201 74.318799) (end 124.477599 74.318799) (width 0.5) (layer F.Cu) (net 15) (status 10))
 (segment (start 120.396 74.748) (end 120.825201 74.318799) (width 0.5) (layer F.Cu) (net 15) (status 30))
 (segment (start 131.39 66.5) (end 131.318 66.428) (width 0.5) (layer B.Cu) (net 2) (status 30))
 (segment (start 133.4 66.5) (end 131.39 66.5) (width 0.5) (layer B.Cu) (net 2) (status 30))
 (segment (start 131.318 67.684) (end 132.08 68.446) (width 0.5) (layer B.Cu) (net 2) (status 20))
 (segment (start 131.318 66.428) (end 131.318 67.684) (width 0.5) (layer B.Cu) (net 2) (status 10))
 (segment (start 133.52 68.446) (end 133.67 68.296) (width 0.5) (layer B.Cu) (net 2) (status 30))
 (segment (start 132.08 68.446) (end 133.52 68.446) (width 0.5) (layer B.Cu) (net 2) (status 30))
 (segment (start 131.179999 69.346001) (end 132.08 68.446) (width 0.5) (layer B.Cu) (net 2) (status 20))
 (segment (start 131.179999 71.776001) (end 131.179999 69.346001) (width 0.5) (layer B.Cu) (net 2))
 (segment (start 133.422999 73.478999) (end 131.790001 71.846001) (width 0.5) (layer B.Cu) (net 2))
 (segment (start 131.790001 71.846001) (end 131.249999 71.846001) (width 0.5) (layer B.Cu) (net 2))
 (segment (start 133.422999 73.809999) (end 133.422999 73.478999) (width 0.5) (layer B.Cu) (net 2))
 (segment (start 131.249999 71.846001) (end 131.179999 71.776001) (width 0.5) (layer B.Cu) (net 2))
 (segment (start 134.223 74.61) (end 133.422999 73.809999) (width 0.5) (layer B.Cu) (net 2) (status 10))
 (segment (start 123 62) (end 129.5 62) (width 0.5) (layer F.Cu) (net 2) (status 30))
 (segment (start 131.318 66.058002) (end 131.318 66.428) (width 0.5) (layer B.Cu) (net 2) (status 30))
 (segment (start 129.5 64.240002) (end 131.318 66.058002) (width 0.5) (layer B.Cu) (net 2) (status 20))
 (segment (start 129.5 62) (end 129.5 64.240002) (width 0.5) (layer B.Cu) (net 2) (status 10))
 (segment (start 130.048 76.832) (end 128.72 78.16) (width 0.5) (layer F.Cu) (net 14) (status 20))
 (segment (start 130.048 75.3488) (end 130.048 76.832) (width 0.5) (layer F.Cu) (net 14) (status 10))
 (segment (start 127.022 84.131) (end 126.899 84.008) (width 0.5) (layer B.Cu) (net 9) (status 30))
 (segment (start 129.794 84.131) (end 127.022 84.131) (width 0.5) (layer B.Cu) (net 9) (status 30))
 (via (at 122.682 78.232) (size 0.8) (drill 0.4) (layers F.Cu B.Cu) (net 8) (status 30))
 (segment (start 135.57 72.182) (end 135.89 72.502) (width 0.5) (layer B.Cu) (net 8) (status 20))
 (segment (start 135.57 70.896) (end 135.57 72.182) (width 0.5) (layer B.Cu) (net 8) (status 10))
 (segment (start 122.682 78.232) (end 122.682 70.866) (width 0.25) (layer B.Cu) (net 8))
 (segment (start 122.682 70.866) (end 122.809 70.739) (width 0.25) (layer B.Cu) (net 8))
 (segment (start 122.809 70.739) (end 129.109 70.739) (width 0.25) (layer B.Cu) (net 8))
 (via (at 129.109 70.739) (size 0.5) (drill 0.3) (layers F.Cu B.Cu) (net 8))
 (segment (start 129.109 70.739) (end 135.459 70.739) (width 0.25) (layer F.Cu) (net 8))
 (via (at 135.459 70.739) (size 0.5) (drill 0.3) (layers F.Cu B.Cu) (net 8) (status 30))
 (segment (start 125.1718 71.247) (end 123.4 73.0188) (width 0.5) (layer F.Cu) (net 4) (status 30))
 (segment (start 125.349 71.247) (end 125.1718 71.247) (width 0.5) (layer F.Cu) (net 4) (status 30))
 (segment (start 123.4 75.48) (end 120.72 78.16) (width 0.5) (layer F.Cu) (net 11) (status 30))
 (segment (start 123.4 75.4188) (end 123.4 75.48) (width 0.5) (layer F.Cu) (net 11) (status 30))
 (via (at 132.207 61.595) (size 0.5) (drill 0.3) (layers F.Cu B.Cu) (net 13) (status 30))
 (via (at 134.239 61.722) (size 0.5) (drill 0.3) (layers F.Cu B.Cu) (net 12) (status 30))
 (segment (start 135.636 68.23) (end 135.57 68.296) (width 0.5) (layer B.Cu) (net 12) (status 30))
 (segment (start 135.636 66.478) (end 135.636 66.548) (width 0.5) (layer B.Cu) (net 12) (status 30))
 (segment (start 135.636 66.548) (end 135.636 68.23) (width 0.5) (layer B.Cu) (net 12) (status 30))
 (via (at 135.636 66.548) (size 0.5) (drill 0.3) (layers F.Cu B.Cu) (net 12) (status 30))
 (segment (start 135.636 66.548) (end 135.636 64.262) (width 0.5) (layer F.Cu) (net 12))
 (segment (start 134.239 62.865) (end 134.239 61.722) (width 0.5) (layer F.Cu) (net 12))
 (segment (start 135.636 64.262) (end 134.239 62.865) (width 0.5) (layer F.Cu) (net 12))
 (segment (start 123 66.5) (end 129.5 66.5) (width 0.5) (layer F.Cu) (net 12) (status 30))
 (segment (start 133.55401 63.54999) (end 134.239 62.865) (width 0.5) (layer F.Cu) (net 12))
 (segment (start 132.45001 63.54999) (end 133.55401 63.54999) (width 0.5) (layer F.Cu) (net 12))
 (segment (start 129.5 66.5) (end 132.45001 63.54999) (width 0.5) (layer F.Cu) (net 12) (status 10))
 (segment (start 127.276 81.731) (end 126.899 82.108) (width 0.5) (layer B.Cu) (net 1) (status 20))
 (segment (start 129.794 81.731) (end 127.276 81.731) (width 0.5) (layer B.Cu) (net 1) (status 10))
 (segment (start 132.223 73.66) (end 133.223 74.66) (width 0.5) (layer B.Cu) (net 1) (status 10))
 (segment (start 133.223 74.66) (end 133.223 76.692616) (width 0.5) (layer B.Cu) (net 1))
 (segment (start 133.223 76.692616) (end 129.794 80.121616) (width 0.5) (layer B.Cu) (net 1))
 (segment (start 129.794 80.121616) (end 129.794 81.731) (width 0.5) (layer B.Cu) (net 1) (status 20))
 (segment (start 134.62 72.313) (end 134.223 72.71) (width 0.5) (layer B.Cu) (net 3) (status 30))
 (segment (start 134.62 70.896) (end 134.62 72.313) (width 0.5) (layer B.Cu) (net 3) (status 30))
 (segment (start 135.023001 73.510001) (end 134.223 72.71) (width 0.5) (layer B.Cu) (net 3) (status 20))
 (segment (start 130.894001 85.668997) (end 128.4765 88.086498) (width 0.5) (layer B.Cu) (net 3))
 (segment (start 135.023001 75.741157) (end 130.894001 79.870157) (width 0.5) (layer B.Cu) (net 3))
 (segment (start 130.894001 79.870157) (end 130.894001 85.668997) (width 0.5) (layer B.Cu) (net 3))
 (segment (start 128.4765 88.086498) (end 128.4765 88.5165) (width 0.5) (layer B.Cu) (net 3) (status 20))
 (segment (start 135.073001 73.560001) (end 135.023001 73.510001) (width 0.4) (layer B.Cu) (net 3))
 (segment (start 135.073001 75.691157) (end 135.073001 73.560001) (width 0.4) (layer B.Cu) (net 3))
 (segment (start 135.023001 75.741157) (end 135.073001 75.691157) (width 0.4) (layer B.Cu) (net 3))
 (via (at 134.112 78.27264) (size 0.5) (drill 0.3) (layers F.Cu B.Cu) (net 6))
 (segment (start 130.4765 87.5665) (end 130.5265 87.5665) (width 0.5) (layer B.Cu) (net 6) (status 30))
 (segment (start 131.494012 86.548988) (end 131.494012 81.675488) (width 0.5) (layer B.Cu) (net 6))
 (segment (start 130.4765 87.5665) (end 131.494012 86.548988) (width 0.5) (layer B.Cu) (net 6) (status 10))
 (segment (start 131.494012 81.675488) (end 133.477 79.6925) (width 0.5) (layer B.Cu) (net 6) (status 20))
 (segment (start 133.37032 79.01432) (end 134.112 78.27264) (width 0.5) (layer B.Cu) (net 6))
 (segment (start 133.37032 79.97384) (end 133.37032 79.01432) (width 0.5) (layer B.Cu) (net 6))
 (segment (start 134.08176 78.89824) (end 133.32 79.66) (width 0.5) (layer F.Cu) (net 6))
 (segment (start 134.08176 78.29804) (end 134.08176 78.89824) (width 0.5) (layer F.Cu) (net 6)))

